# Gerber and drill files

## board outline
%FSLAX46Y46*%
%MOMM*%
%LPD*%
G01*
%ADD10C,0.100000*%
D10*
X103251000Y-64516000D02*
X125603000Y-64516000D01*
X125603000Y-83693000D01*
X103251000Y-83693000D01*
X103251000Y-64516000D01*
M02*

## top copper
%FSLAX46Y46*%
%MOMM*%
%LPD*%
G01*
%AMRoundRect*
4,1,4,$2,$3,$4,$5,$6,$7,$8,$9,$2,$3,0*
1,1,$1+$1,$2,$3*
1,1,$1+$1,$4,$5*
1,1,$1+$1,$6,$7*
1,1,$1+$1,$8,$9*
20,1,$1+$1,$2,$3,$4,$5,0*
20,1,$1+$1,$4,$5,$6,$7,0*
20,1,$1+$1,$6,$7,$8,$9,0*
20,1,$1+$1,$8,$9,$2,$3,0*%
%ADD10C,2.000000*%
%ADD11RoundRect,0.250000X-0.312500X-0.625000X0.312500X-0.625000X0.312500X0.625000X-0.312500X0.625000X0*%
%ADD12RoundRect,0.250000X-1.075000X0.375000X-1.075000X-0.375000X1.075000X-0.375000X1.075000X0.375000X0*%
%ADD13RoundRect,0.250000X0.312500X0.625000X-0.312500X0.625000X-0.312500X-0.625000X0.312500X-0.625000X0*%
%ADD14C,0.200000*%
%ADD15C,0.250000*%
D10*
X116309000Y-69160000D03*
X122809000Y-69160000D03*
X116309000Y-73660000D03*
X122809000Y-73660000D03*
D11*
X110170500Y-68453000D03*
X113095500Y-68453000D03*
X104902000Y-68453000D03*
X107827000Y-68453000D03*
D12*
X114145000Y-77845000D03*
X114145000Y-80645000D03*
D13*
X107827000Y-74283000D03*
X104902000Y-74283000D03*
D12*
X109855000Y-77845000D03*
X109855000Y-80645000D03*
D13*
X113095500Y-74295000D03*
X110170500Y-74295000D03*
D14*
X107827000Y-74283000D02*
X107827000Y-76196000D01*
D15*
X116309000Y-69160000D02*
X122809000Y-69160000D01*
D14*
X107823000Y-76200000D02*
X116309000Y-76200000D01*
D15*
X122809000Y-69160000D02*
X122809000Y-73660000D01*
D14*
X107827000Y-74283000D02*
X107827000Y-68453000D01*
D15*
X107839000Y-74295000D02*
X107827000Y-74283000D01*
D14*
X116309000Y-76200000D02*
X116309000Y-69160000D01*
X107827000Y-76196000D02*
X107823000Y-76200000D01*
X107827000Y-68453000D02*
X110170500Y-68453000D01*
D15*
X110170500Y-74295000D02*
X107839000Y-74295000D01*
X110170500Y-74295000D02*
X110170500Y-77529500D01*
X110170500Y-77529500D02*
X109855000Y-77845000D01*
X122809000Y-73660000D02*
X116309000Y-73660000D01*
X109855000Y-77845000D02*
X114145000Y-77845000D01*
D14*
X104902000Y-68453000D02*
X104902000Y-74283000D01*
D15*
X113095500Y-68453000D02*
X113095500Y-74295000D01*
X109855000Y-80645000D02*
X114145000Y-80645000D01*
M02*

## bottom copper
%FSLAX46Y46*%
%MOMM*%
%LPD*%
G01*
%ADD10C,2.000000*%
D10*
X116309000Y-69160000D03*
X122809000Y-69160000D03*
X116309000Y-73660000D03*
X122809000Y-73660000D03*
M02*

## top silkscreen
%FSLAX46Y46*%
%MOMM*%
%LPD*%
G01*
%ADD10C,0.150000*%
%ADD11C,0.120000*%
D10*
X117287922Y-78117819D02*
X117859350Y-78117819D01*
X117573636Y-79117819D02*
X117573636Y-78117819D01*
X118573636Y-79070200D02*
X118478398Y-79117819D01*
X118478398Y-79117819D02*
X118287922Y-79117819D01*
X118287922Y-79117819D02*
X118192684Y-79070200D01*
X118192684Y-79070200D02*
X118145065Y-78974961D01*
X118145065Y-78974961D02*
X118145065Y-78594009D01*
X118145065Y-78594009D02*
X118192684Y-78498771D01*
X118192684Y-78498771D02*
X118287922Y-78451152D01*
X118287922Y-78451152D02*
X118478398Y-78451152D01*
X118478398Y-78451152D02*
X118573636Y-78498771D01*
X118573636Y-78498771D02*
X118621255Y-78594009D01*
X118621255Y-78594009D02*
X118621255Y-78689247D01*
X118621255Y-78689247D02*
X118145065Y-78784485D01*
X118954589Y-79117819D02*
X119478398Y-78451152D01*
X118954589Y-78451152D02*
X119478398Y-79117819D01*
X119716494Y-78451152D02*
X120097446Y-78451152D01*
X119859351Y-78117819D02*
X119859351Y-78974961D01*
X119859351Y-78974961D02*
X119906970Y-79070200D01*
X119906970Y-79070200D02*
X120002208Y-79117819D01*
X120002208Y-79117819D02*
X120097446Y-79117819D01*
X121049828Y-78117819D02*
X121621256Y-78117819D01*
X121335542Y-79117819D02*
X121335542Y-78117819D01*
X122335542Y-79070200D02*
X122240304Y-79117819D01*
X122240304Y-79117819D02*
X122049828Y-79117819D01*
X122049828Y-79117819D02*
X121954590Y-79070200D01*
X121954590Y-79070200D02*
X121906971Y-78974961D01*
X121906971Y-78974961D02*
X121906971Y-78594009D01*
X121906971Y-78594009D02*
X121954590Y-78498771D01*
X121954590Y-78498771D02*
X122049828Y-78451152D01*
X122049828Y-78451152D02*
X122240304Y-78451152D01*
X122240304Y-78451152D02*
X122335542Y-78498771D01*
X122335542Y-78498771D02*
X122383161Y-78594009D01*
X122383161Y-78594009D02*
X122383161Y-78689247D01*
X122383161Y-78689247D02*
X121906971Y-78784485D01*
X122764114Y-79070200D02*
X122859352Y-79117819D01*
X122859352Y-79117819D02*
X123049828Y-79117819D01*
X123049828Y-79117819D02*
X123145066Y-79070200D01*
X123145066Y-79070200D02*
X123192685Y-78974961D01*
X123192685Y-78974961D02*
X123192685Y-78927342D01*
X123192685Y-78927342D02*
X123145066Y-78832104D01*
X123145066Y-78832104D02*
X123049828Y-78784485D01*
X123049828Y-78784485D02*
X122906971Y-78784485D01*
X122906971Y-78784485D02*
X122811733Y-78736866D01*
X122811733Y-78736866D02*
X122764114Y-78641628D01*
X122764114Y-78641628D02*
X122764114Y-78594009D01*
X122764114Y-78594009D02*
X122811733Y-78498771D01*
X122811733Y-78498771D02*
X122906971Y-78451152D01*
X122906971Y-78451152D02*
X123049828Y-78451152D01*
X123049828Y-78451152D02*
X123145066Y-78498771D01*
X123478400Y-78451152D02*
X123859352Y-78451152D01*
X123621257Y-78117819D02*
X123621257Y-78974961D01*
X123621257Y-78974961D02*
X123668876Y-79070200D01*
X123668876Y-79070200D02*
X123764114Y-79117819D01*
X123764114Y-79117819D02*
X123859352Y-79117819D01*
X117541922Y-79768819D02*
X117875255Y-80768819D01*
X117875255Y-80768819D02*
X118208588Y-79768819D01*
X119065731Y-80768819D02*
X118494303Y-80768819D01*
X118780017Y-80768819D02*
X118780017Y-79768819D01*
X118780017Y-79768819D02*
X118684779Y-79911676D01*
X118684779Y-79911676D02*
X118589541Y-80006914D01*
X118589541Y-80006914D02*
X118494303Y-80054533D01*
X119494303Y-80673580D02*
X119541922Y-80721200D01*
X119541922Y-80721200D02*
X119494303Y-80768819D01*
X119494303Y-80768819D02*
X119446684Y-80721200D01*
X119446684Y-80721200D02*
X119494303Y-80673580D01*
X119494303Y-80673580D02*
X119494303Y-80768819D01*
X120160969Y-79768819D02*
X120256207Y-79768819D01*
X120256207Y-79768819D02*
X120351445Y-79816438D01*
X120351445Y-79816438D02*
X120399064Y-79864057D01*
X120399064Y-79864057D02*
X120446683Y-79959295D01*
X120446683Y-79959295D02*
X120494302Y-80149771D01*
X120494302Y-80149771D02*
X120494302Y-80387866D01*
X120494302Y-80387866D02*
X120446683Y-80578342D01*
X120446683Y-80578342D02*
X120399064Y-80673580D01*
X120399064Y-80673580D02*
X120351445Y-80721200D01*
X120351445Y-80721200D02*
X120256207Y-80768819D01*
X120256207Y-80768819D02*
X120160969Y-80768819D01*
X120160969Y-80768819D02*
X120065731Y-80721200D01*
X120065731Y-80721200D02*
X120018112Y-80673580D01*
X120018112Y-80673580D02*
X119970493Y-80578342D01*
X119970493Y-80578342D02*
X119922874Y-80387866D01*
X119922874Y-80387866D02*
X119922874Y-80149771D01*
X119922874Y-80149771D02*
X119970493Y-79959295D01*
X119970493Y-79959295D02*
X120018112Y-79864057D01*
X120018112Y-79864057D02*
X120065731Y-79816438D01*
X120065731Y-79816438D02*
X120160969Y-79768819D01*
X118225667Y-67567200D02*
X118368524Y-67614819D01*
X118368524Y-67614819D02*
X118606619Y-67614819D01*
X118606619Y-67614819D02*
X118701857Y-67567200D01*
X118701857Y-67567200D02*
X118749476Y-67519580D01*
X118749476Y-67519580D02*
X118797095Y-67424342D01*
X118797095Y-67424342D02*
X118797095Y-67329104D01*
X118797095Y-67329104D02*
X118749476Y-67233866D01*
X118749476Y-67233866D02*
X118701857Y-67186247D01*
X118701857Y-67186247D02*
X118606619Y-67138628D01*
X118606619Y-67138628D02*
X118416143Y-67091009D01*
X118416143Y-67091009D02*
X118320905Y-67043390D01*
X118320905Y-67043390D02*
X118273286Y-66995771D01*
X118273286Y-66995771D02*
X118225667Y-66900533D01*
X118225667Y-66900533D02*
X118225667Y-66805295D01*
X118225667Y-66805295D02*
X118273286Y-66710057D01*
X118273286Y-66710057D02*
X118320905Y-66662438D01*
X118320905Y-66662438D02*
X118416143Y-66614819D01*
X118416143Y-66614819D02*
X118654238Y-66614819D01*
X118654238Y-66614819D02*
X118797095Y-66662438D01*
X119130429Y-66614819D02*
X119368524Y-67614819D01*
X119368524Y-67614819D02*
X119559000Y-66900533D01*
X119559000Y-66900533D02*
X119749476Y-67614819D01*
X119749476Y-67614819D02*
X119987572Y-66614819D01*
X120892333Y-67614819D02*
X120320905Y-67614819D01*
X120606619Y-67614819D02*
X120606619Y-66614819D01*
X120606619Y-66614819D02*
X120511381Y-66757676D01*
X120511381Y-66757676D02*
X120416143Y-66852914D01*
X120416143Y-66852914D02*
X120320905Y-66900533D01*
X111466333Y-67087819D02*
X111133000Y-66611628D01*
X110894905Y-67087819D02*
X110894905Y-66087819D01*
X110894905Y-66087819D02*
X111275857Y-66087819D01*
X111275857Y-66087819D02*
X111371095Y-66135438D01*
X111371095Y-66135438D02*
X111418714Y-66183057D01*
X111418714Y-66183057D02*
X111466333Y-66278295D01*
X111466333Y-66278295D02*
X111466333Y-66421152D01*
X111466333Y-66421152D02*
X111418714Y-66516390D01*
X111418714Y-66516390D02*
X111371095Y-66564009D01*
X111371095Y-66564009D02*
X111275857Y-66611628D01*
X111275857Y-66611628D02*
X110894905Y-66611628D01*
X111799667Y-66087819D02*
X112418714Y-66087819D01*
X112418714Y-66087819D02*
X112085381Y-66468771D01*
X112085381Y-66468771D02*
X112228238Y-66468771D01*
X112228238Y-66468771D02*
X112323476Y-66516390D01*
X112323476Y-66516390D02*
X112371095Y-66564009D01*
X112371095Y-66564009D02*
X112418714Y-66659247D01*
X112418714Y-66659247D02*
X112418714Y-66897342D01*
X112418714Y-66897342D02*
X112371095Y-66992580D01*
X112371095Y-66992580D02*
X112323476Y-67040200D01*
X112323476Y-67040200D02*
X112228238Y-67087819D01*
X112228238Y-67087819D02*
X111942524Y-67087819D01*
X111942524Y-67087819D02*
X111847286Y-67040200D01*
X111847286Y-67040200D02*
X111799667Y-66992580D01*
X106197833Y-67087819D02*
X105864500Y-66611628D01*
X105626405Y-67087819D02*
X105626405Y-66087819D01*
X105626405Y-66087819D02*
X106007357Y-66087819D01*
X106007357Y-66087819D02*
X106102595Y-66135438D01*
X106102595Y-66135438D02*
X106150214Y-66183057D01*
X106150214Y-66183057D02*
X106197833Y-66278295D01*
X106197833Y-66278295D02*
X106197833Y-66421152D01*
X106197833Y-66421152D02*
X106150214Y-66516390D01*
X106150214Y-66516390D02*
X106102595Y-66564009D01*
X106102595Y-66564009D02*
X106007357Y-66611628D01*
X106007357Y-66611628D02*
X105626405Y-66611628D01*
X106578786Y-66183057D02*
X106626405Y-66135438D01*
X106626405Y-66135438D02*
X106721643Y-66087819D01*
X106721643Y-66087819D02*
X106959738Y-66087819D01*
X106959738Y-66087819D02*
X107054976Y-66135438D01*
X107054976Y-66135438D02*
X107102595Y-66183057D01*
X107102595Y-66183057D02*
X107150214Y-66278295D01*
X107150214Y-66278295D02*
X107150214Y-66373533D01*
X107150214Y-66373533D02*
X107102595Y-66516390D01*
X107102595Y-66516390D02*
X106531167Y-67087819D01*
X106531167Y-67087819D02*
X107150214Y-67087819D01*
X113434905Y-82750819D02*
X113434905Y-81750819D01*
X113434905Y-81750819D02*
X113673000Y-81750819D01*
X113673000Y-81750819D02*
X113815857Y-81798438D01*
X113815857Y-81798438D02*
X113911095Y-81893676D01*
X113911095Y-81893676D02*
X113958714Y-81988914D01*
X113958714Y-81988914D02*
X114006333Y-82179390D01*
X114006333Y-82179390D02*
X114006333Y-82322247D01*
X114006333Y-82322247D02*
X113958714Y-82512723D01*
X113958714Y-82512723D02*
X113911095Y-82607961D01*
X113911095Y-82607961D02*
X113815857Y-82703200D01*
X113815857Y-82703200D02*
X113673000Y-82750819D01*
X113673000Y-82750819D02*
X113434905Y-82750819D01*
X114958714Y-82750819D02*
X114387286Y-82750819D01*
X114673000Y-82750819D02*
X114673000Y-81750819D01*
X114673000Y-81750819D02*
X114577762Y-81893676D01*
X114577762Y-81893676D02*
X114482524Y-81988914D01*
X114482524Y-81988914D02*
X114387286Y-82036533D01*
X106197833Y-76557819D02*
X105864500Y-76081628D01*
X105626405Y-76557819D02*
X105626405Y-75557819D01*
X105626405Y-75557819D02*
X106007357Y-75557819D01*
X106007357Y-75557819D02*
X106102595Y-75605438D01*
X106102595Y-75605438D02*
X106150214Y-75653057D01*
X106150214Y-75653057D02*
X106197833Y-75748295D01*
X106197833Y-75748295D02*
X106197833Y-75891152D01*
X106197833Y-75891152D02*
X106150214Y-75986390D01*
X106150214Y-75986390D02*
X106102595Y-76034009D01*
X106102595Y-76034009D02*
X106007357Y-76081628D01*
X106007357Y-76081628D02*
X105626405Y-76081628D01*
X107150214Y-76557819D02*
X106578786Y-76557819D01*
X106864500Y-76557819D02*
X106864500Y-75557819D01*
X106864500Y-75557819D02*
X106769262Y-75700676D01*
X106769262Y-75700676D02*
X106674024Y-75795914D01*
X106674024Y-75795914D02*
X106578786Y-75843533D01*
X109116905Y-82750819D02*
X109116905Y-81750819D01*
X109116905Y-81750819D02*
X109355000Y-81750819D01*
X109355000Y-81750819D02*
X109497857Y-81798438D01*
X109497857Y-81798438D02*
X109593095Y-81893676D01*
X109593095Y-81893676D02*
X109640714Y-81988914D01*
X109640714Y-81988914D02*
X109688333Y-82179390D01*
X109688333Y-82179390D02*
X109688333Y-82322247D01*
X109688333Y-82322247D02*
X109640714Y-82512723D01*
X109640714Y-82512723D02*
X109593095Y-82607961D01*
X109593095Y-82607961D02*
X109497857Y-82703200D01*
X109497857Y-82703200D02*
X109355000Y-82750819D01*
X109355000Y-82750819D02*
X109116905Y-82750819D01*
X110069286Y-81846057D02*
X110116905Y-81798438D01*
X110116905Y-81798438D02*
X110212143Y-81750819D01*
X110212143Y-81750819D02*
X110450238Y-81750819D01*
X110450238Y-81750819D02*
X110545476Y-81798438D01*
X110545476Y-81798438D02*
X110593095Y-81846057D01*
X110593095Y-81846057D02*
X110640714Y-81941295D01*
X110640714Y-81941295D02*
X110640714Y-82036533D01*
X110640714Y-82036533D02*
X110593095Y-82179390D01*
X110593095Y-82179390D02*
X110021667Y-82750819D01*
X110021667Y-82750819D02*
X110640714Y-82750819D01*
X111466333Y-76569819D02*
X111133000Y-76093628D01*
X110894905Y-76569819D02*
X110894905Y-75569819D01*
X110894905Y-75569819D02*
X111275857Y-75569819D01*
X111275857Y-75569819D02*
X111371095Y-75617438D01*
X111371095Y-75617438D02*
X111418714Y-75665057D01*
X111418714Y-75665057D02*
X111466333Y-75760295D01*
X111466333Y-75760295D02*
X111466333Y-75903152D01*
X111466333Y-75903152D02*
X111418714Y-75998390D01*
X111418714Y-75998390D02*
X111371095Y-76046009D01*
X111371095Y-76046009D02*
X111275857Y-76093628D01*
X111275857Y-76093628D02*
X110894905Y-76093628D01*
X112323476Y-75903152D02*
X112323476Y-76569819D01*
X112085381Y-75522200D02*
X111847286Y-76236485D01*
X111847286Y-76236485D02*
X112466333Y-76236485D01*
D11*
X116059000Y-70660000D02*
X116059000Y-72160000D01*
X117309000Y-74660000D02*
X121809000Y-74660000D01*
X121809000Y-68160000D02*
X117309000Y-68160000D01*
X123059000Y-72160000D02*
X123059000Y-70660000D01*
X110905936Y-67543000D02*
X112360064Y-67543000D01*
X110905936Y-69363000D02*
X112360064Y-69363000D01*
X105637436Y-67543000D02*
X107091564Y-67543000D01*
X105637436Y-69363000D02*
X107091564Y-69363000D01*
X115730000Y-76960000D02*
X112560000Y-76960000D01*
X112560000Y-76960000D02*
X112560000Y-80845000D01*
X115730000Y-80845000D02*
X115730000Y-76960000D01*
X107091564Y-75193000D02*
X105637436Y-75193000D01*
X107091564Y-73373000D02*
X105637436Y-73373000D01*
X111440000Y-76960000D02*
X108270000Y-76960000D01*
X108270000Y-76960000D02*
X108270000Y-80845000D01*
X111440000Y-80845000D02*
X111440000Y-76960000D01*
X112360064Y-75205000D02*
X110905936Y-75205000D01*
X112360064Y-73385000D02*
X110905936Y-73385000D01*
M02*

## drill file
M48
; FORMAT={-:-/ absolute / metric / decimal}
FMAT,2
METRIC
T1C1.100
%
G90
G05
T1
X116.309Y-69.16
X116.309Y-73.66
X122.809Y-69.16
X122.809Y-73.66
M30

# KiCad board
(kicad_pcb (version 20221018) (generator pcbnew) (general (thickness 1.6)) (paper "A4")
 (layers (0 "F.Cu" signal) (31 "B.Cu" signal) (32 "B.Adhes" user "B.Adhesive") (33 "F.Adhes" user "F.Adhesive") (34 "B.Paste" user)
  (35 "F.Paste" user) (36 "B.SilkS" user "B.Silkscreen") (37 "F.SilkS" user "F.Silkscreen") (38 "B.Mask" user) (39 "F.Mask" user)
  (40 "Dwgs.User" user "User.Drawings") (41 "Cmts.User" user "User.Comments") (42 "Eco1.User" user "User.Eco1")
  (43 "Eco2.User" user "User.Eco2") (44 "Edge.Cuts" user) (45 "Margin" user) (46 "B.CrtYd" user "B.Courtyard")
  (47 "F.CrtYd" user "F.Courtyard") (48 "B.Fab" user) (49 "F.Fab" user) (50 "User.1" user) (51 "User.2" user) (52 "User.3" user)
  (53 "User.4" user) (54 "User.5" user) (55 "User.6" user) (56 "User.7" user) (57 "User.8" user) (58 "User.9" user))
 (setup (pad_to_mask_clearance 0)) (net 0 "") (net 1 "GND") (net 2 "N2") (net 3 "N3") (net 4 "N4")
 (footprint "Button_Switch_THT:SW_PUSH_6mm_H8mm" (layer "F.Cu") (at 116.309 69.16)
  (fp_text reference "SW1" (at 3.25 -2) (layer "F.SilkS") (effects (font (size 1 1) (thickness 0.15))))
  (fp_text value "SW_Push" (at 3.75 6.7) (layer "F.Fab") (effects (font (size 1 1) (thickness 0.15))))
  (fp_line (start -0.25 1.5) (end -0.25 3) (stroke (width 0.12) (type solid)) (layer "F.SilkS"))
  (fp_line (start 1 5.5) (end 5.5 5.5) (stroke (width 0.12) (type solid)) (layer "F.SilkS"))
  (fp_line (start 5.5 -1) (end 1 -1) (stroke (width 0.12) (type solid)) (layer "F.SilkS"))
  (fp_line (start 6.75 3) (end 6.75 1.5) (stroke (width 0.12) (type solid)) (layer "F.SilkS"))
  (pad "1" thru_hole circle (at 0 0 90) (size 2 2) (drill 1.1) (layers "*.Cu" "*.Mask") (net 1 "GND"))
  (pad "1" thru_hole circle (at 6.5 0 90) (size 2 2) (drill 1.1) (layers "*.Cu" "*.Mask") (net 1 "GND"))
  (pad "2" thru_hole circle (at 0 4.5 90) (size 2 2) (drill 1.1) (layers "*.Cu" "*.Mask") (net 1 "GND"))
  (pad "2" thru_hole circle (at 6.5 4.5 90) (size 2 2) (drill 1.1) (layers "*.Cu" "*.Mask") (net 1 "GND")))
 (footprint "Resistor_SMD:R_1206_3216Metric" (layer "F.Cu") (at 111.633 68.453)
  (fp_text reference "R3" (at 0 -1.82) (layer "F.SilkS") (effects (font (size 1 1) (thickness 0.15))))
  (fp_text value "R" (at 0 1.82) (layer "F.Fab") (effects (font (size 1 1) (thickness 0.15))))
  (fp_line (start -0.727064 -0.91) (end 0.727064 -0.91) (stroke (width 0.12) (type solid)) (layer "F.SilkS"))
  (fp_line (start -0.727064 0.91) (end 0.727064 0.91) (stroke (width 0.12) (type solid)) (layer "F.SilkS"))
  (pad "1" smd roundrect (at -1.4625 0) (size 1.125 1.75) (layers "F.Cu" "F.Paste" "F.Mask") (roundrect_rratio 0.222222) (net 1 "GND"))
  (pad "2" smd roundrect (at 1.4625 0) (size 1.125 1.75) (layers "F.Cu" "F.Paste" "F.Mask") (roundrect_rratio 0.222222) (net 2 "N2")))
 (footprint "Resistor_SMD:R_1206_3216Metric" (layer "F.Cu") (at 106.3645 68.453)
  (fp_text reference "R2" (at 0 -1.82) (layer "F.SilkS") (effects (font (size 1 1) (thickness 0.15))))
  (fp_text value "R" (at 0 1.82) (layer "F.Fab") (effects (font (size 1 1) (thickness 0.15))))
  (fp_line (start -0.727064 -0.91) (end 0.727064 -0.91) (stroke (width 0.12) (type solid)) (layer "F.SilkS"))
  (fp_line (start -0.727064 0.91) (end 0.727064 0.91) (stroke (width 0.12) (type solid)) (layer "F.SilkS"))
  (pad "1" smd roundrect (at -1.4625 0) (size 1.125 1.75) (layers "F.Cu" "F.Paste" "F.Mask") (roundrect_rratio 0.222222) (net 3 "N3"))
  (pad "2" smd roundrect (at 1.4625 0) (size 1.125 1.75) (layers "F.Cu" "F.Paste" "F.Mask") (roundrect_rratio 0.222222) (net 1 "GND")))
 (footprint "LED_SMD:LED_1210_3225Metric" (layer "F.Cu") (at 114.145 79.245 -90)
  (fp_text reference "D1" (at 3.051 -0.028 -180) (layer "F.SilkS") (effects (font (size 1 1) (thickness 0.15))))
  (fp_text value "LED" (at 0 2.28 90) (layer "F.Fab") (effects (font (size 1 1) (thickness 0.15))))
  (fp_line (start -2.285 -1.585) (end -2.285 1.585) (stroke (width 0.12) (type solid)) (layer "F.SilkS"))
  (fp_line (start -2.285 1.585) (end 1.6 1.585) (stroke (width 0.12) (type solid)) (layer "F.SilkS"))
  (fp_line (start 1.6 -1.585) (end -2.285 -1.585) (stroke (width 0.12) (type solid)) (layer "F.SilkS"))
  (pad "1" smd roundrect (at -1.4 0 270) (size 1.25 2.65) (layers "F.Cu" "F.Paste" "F.Mask") (roundrect_rratio 0.2) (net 1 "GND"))
  (pad "2" smd roundrect (at 1.4 0 270) (size 1.25 2.65) (layers "F.Cu" "F.Paste" "F.Mask") (roundrect_rratio 0.2) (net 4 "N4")))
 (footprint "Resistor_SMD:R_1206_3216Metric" (layer "F.Cu") (at 106.3645 74.283 180)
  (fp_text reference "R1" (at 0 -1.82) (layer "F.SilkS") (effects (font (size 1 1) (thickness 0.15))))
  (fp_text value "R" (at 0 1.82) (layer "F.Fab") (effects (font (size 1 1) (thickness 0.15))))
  (fp_line (start -0.727064 -0.91) (end 0.727064 -0.91) (stroke (width 0.12) (type solid)) (layer "F.SilkS"))
  (fp_line (start -0.727064 0.91) (end 0.727064 0.91) (stroke (width 0.12) (type solid)) (layer "F.SilkS"))
  (pad "1" smd roundrect (at -1.4625 0 180) (size 1.125 1.75) (layers "F.Cu" "F.Paste" "F.Mask") (roundrect_rratio 0.222222) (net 1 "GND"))
  (pad "2" smd roundrect (at 1.4625 0 180) (size 1.125 1.75) (layers "F.Cu" "F.Paste" "F.Mask") (roundrect_rratio 0.222222) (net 3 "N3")))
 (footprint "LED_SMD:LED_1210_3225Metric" (layer "F.Cu") (at 109.855 79.245 -90)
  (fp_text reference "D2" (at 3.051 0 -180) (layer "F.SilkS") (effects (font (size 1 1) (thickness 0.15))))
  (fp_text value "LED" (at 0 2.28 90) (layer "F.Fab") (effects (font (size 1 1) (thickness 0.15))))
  (fp_line (start -2.285 -1.585) (end -2.285 1.585) (stroke (width 0.12) (type solid)) (layer "F.SilkS"))
  (fp_line (start -2.285 1.585) (end 1.6 1.585) (stroke (width 0.12) (type solid)) (layer "F.SilkS"))
  (fp_line (start 1.6 -1.585) (end -2.285 -1.585) (stroke (width 0.12) (type solid)) (layer "F.SilkS"))
  (pad "1" smd roundrect (at -1.4 0 270) (size 1.25 2.65) (layers "F.Cu" "F.Paste" "F.Mask") (roundrect_rratio 0.2) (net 1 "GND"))
  (pad "2" smd roundrect (at 1.4 0 270) (size 1.25 2.65) (layers "F.Cu" "F.Paste" "F.Mask") (roundrect_rratio 0.2) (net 4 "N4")))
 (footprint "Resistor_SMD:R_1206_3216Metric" (layer "F.Cu") (at 111.633 74.295 180)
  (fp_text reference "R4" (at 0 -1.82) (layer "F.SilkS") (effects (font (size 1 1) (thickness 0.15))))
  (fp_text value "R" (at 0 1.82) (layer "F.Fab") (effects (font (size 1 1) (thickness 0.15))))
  (fp_line (start -0.727064 -0.91) (end 0.727064 -0.91) (stroke (width 0.12) (type solid)) (layer "F.SilkS"))
  (fp_line (start -0.727064 0.91) (end 0.727064 0.91) (stroke (width 0.12) (type solid)) (layer "F.SilkS"))
  (pad "1" smd roundrect (at -1.4625 0 180) (size 1.125 1.75) (layers "F.Cu" "F.Paste" "F.Mask") (roundrect_rratio 0.222222) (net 2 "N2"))
  (pad "2" smd roundrect (at 1.4625 0 180) (size 1.125 1.75) (layers "F.Cu" "F.Paste" "F.Mask") (roundrect_rratio 0.222222) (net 1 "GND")))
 (gr_rect (start 103.251 64.516) (end 125.603 83.693) (stroke (width 0.1) (type default)) (fill none) (layer "Edge.Cuts"))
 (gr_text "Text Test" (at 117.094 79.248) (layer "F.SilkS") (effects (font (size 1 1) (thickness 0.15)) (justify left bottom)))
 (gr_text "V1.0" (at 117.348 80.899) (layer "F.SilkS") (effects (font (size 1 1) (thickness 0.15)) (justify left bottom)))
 (segment (start 107.827 74.283) (end 107.827 76.196) (width 0.2) (layer "F.Cu") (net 1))
 (segment (start 116.309 69.16) (end 122.809 69.16) (width 0.25) (layer "F.Cu") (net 1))
 (segment (start 107.823 76.2) (end 116.309 76.2) (width 0.2) (layer "F.Cu") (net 1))
 (segment (start 122.809 69.16) (end 122.809 73.66) (width 0.25) (layer "F.Cu") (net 1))
 (segment (start 107.827 74.283) (end 107.827 68.453) (width 0.2) (layer "F.Cu") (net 1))
 (segment (start 107.839 74.295) (end 107.827 74.283) (width 0.25) (layer "F.Cu") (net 1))
 (segment (start 116.309 76.2) (end 116.309 69.16) (width 0.2) (layer "F.Cu") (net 1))
 (segment (start 107.827 76.196) (end 107.823 76.2) (width 0.2) (layer "F.Cu") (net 1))
 (segment (start 107.827 68.453) (end 110.1705 68.453) (width 0.2) (layer "F.Cu") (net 1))
 (segment (start 110.1705 74.295) (end 107.839 74.295) (width 0.25) (layer "F.Cu") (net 1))
 (segment (start 110.1705 74.295) (end 110.1705 77.5295) (width 0.25) (layer "F.Cu") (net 1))
 (segment (start 110.1705 77.5295) (end 109.855 77.845) (width 0.25) (layer "F.Cu") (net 1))
 (segment (start 122.809 73.66) (end 116.309 73.66) (width 0.25) (layer "F.Cu") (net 1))
 (segment (start 109.855 77.845) (end 114.145 77.845) (width 0.25) (layer "F.Cu") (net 1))
 (segment (start 104.902 68.453) (end 104.902 74.283) (width 0.2) (layer "F.Cu") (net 3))
 (segment (start 113.0955 68.453) (end 113.0955 74.295) (width 0.25) (layer "F.Cu") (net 2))
 (segment (start 109.855 80.645) (end 114.145 80.645) (width 0.25) (layer "F.Cu") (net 4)))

